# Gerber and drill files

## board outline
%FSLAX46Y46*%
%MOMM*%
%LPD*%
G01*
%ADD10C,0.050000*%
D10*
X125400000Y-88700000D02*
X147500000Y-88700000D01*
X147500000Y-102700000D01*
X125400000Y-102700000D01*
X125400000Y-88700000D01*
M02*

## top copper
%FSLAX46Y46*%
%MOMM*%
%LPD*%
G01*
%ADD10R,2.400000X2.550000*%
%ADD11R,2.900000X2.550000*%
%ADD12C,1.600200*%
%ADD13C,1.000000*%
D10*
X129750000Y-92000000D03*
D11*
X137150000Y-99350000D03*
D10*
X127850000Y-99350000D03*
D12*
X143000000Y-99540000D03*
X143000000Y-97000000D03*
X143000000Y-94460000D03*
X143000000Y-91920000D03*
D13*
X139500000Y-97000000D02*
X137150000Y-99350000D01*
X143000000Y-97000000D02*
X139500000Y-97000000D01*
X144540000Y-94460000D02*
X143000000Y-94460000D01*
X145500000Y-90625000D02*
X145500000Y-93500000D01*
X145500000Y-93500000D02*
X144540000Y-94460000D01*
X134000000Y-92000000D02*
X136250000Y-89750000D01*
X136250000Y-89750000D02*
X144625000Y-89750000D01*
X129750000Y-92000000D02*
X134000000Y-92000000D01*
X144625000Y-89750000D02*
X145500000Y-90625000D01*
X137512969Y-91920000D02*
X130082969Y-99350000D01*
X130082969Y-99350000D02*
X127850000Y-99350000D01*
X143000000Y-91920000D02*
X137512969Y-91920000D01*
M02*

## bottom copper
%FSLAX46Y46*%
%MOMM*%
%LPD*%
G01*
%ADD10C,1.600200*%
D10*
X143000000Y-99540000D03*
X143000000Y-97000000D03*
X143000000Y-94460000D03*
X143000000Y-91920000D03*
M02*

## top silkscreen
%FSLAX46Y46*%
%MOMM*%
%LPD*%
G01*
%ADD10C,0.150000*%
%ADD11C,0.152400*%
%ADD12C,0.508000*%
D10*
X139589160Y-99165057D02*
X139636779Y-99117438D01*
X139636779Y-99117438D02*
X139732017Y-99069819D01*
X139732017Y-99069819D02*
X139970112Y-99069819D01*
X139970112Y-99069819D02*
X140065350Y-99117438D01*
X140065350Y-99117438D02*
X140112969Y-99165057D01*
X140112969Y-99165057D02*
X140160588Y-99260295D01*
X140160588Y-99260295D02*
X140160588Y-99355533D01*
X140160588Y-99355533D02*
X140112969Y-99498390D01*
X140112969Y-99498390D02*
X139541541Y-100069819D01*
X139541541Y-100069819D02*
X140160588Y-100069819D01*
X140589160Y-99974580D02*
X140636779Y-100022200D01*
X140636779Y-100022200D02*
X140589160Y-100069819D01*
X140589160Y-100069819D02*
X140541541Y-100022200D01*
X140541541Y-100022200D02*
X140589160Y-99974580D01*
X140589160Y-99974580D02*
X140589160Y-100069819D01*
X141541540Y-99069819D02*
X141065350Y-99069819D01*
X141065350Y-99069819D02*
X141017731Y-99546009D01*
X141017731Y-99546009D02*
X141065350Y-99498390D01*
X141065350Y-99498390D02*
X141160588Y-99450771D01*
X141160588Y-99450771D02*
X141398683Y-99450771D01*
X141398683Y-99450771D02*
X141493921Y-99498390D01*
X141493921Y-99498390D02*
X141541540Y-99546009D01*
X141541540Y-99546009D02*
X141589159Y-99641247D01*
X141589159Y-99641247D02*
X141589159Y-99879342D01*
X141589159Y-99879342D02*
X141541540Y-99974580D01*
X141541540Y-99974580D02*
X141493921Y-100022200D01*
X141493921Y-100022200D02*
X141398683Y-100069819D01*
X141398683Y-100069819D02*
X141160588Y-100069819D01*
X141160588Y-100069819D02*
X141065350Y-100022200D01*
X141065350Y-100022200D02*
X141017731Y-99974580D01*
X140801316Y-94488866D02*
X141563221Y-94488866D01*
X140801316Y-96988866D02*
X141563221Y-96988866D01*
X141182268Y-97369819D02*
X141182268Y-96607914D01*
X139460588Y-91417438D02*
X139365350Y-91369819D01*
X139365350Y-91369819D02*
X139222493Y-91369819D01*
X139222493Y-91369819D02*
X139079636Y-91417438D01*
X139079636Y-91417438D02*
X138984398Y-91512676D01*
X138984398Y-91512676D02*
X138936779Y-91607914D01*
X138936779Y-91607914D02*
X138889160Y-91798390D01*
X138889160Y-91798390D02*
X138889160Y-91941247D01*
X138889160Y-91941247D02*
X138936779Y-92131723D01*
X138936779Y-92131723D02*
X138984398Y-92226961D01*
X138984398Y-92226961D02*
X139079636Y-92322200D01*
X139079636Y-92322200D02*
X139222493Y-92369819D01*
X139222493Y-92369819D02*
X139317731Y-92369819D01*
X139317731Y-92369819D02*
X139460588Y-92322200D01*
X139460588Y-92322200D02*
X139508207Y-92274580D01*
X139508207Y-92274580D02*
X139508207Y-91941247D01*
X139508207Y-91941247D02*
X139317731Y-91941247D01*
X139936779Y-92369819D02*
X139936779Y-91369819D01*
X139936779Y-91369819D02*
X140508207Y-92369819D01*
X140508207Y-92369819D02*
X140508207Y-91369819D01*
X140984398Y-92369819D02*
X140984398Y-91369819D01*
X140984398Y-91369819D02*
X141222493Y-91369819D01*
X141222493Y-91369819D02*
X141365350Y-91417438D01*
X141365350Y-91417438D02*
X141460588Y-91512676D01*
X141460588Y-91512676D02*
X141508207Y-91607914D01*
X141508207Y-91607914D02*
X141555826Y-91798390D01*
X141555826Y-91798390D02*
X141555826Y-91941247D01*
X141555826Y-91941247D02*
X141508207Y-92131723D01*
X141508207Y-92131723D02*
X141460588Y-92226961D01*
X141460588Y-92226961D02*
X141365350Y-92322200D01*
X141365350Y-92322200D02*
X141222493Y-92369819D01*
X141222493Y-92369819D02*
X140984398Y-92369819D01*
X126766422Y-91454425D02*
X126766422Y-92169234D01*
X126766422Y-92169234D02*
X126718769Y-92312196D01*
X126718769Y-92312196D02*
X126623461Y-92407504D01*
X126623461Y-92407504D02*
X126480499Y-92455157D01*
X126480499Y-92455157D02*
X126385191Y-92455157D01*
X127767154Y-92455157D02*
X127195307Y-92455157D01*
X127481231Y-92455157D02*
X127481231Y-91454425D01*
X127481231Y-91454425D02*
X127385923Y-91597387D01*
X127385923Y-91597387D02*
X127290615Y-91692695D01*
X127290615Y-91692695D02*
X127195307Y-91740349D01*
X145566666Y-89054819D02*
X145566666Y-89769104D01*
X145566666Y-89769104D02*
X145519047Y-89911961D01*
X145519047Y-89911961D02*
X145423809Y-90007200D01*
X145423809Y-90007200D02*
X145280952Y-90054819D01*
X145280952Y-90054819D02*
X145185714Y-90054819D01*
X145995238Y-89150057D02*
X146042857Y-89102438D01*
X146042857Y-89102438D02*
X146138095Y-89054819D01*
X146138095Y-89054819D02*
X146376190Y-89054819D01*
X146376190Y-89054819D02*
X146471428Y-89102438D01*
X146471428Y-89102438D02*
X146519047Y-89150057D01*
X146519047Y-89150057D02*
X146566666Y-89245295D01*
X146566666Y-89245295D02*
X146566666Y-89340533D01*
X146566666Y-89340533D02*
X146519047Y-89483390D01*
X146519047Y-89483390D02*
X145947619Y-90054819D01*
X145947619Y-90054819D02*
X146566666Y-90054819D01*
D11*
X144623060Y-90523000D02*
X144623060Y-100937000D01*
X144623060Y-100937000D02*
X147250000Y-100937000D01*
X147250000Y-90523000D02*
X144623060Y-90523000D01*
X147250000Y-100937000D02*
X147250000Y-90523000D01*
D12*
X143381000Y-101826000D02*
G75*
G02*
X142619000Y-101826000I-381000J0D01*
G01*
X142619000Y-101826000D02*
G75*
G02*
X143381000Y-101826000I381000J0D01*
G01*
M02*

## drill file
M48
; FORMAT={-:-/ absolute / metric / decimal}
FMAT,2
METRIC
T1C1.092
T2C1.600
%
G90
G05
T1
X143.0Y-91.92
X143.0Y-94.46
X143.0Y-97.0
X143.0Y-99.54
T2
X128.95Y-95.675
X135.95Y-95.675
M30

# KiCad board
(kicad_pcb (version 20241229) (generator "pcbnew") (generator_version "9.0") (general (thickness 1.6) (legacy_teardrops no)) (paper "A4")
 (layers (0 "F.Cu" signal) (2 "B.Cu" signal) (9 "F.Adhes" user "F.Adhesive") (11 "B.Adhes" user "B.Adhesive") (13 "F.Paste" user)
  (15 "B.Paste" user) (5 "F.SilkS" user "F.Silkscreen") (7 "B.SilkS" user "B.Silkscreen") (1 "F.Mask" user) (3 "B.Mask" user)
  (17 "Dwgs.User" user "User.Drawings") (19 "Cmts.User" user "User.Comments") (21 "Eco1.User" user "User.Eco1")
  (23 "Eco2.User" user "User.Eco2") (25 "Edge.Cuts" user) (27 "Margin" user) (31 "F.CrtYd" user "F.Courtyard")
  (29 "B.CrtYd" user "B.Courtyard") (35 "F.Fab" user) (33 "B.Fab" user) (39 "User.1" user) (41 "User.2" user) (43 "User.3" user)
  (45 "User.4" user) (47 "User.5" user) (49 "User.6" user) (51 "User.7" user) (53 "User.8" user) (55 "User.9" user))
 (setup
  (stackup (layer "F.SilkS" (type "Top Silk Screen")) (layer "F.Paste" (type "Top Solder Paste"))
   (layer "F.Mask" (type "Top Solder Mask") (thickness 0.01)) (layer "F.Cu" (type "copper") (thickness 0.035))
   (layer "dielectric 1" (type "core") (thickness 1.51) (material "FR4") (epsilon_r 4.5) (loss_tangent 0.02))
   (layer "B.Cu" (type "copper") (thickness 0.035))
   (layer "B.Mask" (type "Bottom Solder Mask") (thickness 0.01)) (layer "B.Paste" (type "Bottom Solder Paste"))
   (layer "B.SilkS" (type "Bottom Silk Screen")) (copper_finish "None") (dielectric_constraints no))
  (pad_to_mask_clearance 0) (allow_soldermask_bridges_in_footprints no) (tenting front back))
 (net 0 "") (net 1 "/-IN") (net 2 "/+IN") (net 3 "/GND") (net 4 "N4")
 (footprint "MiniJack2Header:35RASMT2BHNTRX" (layer "F.Cu") (at 132.45 95.675)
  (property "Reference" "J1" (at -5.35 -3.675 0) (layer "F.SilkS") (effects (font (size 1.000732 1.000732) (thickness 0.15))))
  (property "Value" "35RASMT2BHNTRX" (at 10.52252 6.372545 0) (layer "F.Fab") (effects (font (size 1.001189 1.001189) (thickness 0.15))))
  (pad "" np_thru_hole circle (at -3.5 0) (size 1.6 1.6) (drill 1.6) (layers "*.Cu" "*.Mask"))
  (pad "" np_thru_hole circle (at 3.5 0) (size 1.6 1.6) (drill 1.6) (layers "*.Cu" "*.Mask"))
  (pad "1" smd rect (at -2.7 -3.675) (size 2.4 2.55) (layers "F.Cu" "F.Mask" "F.Paste") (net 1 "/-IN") (solder_mask_margin 0.102))
  (pad "4" smd rect (at 4.7 3.675) (size 2.9 2.55) (layers "F.Cu" "F.Mask" "F.Paste") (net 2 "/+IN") (solder_mask_margin 0.102))
  (pad "5" smd rect (at -4.6 3.675) (size 2.4 2.55) (layers "F.Cu" "F.Mask" "F.Paste") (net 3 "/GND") (solder_mask_margin 0.102)))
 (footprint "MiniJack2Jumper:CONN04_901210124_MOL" (layer "F.Cu") (at 143 99.54 90)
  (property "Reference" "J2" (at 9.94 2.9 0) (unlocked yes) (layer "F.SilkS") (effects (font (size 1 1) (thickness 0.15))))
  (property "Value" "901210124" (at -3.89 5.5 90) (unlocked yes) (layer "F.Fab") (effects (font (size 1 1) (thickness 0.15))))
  (fp_line (start 9.017 1.62306) (end -1.397 1.62306) (stroke (width 0.1524) (type solid)) (layer "F.SilkS"))
  (fp_line (start -1.397 1.62306) (end -1.397 4.25) (stroke (width 0.1524) (type solid)) (layer "F.SilkS"))
  (fp_line (start 9.017 4.25) (end 9.017 1.62306) (stroke (width 0.1524) (type solid)) (layer "F.SilkS"))
  (fp_line (start -1.397 4.25) (end 9.017 4.25) (stroke (width 0.1524) (type solid)) (layer "F.SilkS"))
  (fp_circle (center -2.286 0) (end -1.905 0) (stroke (width 0.508) (type solid)) (fill no) (layer "F.SilkS"))
  (pad "1" thru_hole circle (at 0 0 90) (size 1.6002 1.6002) (drill 1.0922) (layers "*.Cu" "*.Mask") (remove_unused_layers no) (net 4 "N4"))
  (pad "2" thru_hole circle (at 2.54 0 90) (size 1.6002 1.6002) (drill 1.0922) (layers "*.Cu" "*.Mask") (remove_unused_layers no)
   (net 2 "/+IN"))
  (pad "3" thru_hole circle (at 5.08 0 90) (size 1.6002 1.6002) (drill 1.0922) (layers "*.Cu" "*.Mask") (remove_unused_layers no)
   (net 1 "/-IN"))
  (pad "4" thru_hole circle (at 7.62 0 90) (size 1.6002 1.6002) (drill 1.0922) (layers "*.Cu" "*.Mask") (remove_unused_layers no)
   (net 3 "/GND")))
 (gr_rect (start 125.4 88.7) (end 147.5 102.7) (stroke (width 0.05) (type default)) (fill no) (layer "Edge.Cuts"))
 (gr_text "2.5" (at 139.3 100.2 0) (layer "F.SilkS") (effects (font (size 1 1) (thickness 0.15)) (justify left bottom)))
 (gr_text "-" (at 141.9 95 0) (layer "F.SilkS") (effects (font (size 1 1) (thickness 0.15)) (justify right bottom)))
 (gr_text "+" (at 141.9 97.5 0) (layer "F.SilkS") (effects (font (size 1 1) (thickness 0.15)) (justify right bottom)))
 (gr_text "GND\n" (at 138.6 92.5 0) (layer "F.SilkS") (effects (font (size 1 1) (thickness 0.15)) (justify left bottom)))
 (segment (start 143 97) (end 139.5 97) (width 1) (layer "F.Cu") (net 2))
 (segment (start 139.5 97) (end 137.15 99.35) (width 1) (layer "F.Cu") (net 2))
 (segment (start 137.512969 91.92) (end 130.082969 99.35) (width 1) (layer "F.Cu") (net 3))
 (segment (start 130.082969 99.35) (end 127.85 99.35) (width 1) (layer "F.Cu") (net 3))
 (segment (start 143 91.92) (end 137.512969 91.92) (width 1) (layer "F.Cu") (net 3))
 (segment (start 145.5 90.625) (end 145.5 93.5) (width 1) (layer "F.Cu") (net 1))
 (segment (start 144.54 94.46) (end 143 94.46) (width 1) (layer "F.Cu") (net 1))
 (segment (start 136.25 89.75) (end 144.625 89.75) (width 1) (layer "F.Cu") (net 1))
 (segment (start 145.5 93.5) (end 144.54 94.46) (width 1) (layer "F.Cu") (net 1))
 (segment (start 144.625 89.75) (end 145.5 90.625) (width 1) (layer "F.Cu") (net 1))
 (segment (start 129.75 92) (end 134 92) (width 1) (layer "F.Cu") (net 1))
 (segment (start 134 92) (end 136.25 89.75) (width 1) (layer "F.Cu") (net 1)))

